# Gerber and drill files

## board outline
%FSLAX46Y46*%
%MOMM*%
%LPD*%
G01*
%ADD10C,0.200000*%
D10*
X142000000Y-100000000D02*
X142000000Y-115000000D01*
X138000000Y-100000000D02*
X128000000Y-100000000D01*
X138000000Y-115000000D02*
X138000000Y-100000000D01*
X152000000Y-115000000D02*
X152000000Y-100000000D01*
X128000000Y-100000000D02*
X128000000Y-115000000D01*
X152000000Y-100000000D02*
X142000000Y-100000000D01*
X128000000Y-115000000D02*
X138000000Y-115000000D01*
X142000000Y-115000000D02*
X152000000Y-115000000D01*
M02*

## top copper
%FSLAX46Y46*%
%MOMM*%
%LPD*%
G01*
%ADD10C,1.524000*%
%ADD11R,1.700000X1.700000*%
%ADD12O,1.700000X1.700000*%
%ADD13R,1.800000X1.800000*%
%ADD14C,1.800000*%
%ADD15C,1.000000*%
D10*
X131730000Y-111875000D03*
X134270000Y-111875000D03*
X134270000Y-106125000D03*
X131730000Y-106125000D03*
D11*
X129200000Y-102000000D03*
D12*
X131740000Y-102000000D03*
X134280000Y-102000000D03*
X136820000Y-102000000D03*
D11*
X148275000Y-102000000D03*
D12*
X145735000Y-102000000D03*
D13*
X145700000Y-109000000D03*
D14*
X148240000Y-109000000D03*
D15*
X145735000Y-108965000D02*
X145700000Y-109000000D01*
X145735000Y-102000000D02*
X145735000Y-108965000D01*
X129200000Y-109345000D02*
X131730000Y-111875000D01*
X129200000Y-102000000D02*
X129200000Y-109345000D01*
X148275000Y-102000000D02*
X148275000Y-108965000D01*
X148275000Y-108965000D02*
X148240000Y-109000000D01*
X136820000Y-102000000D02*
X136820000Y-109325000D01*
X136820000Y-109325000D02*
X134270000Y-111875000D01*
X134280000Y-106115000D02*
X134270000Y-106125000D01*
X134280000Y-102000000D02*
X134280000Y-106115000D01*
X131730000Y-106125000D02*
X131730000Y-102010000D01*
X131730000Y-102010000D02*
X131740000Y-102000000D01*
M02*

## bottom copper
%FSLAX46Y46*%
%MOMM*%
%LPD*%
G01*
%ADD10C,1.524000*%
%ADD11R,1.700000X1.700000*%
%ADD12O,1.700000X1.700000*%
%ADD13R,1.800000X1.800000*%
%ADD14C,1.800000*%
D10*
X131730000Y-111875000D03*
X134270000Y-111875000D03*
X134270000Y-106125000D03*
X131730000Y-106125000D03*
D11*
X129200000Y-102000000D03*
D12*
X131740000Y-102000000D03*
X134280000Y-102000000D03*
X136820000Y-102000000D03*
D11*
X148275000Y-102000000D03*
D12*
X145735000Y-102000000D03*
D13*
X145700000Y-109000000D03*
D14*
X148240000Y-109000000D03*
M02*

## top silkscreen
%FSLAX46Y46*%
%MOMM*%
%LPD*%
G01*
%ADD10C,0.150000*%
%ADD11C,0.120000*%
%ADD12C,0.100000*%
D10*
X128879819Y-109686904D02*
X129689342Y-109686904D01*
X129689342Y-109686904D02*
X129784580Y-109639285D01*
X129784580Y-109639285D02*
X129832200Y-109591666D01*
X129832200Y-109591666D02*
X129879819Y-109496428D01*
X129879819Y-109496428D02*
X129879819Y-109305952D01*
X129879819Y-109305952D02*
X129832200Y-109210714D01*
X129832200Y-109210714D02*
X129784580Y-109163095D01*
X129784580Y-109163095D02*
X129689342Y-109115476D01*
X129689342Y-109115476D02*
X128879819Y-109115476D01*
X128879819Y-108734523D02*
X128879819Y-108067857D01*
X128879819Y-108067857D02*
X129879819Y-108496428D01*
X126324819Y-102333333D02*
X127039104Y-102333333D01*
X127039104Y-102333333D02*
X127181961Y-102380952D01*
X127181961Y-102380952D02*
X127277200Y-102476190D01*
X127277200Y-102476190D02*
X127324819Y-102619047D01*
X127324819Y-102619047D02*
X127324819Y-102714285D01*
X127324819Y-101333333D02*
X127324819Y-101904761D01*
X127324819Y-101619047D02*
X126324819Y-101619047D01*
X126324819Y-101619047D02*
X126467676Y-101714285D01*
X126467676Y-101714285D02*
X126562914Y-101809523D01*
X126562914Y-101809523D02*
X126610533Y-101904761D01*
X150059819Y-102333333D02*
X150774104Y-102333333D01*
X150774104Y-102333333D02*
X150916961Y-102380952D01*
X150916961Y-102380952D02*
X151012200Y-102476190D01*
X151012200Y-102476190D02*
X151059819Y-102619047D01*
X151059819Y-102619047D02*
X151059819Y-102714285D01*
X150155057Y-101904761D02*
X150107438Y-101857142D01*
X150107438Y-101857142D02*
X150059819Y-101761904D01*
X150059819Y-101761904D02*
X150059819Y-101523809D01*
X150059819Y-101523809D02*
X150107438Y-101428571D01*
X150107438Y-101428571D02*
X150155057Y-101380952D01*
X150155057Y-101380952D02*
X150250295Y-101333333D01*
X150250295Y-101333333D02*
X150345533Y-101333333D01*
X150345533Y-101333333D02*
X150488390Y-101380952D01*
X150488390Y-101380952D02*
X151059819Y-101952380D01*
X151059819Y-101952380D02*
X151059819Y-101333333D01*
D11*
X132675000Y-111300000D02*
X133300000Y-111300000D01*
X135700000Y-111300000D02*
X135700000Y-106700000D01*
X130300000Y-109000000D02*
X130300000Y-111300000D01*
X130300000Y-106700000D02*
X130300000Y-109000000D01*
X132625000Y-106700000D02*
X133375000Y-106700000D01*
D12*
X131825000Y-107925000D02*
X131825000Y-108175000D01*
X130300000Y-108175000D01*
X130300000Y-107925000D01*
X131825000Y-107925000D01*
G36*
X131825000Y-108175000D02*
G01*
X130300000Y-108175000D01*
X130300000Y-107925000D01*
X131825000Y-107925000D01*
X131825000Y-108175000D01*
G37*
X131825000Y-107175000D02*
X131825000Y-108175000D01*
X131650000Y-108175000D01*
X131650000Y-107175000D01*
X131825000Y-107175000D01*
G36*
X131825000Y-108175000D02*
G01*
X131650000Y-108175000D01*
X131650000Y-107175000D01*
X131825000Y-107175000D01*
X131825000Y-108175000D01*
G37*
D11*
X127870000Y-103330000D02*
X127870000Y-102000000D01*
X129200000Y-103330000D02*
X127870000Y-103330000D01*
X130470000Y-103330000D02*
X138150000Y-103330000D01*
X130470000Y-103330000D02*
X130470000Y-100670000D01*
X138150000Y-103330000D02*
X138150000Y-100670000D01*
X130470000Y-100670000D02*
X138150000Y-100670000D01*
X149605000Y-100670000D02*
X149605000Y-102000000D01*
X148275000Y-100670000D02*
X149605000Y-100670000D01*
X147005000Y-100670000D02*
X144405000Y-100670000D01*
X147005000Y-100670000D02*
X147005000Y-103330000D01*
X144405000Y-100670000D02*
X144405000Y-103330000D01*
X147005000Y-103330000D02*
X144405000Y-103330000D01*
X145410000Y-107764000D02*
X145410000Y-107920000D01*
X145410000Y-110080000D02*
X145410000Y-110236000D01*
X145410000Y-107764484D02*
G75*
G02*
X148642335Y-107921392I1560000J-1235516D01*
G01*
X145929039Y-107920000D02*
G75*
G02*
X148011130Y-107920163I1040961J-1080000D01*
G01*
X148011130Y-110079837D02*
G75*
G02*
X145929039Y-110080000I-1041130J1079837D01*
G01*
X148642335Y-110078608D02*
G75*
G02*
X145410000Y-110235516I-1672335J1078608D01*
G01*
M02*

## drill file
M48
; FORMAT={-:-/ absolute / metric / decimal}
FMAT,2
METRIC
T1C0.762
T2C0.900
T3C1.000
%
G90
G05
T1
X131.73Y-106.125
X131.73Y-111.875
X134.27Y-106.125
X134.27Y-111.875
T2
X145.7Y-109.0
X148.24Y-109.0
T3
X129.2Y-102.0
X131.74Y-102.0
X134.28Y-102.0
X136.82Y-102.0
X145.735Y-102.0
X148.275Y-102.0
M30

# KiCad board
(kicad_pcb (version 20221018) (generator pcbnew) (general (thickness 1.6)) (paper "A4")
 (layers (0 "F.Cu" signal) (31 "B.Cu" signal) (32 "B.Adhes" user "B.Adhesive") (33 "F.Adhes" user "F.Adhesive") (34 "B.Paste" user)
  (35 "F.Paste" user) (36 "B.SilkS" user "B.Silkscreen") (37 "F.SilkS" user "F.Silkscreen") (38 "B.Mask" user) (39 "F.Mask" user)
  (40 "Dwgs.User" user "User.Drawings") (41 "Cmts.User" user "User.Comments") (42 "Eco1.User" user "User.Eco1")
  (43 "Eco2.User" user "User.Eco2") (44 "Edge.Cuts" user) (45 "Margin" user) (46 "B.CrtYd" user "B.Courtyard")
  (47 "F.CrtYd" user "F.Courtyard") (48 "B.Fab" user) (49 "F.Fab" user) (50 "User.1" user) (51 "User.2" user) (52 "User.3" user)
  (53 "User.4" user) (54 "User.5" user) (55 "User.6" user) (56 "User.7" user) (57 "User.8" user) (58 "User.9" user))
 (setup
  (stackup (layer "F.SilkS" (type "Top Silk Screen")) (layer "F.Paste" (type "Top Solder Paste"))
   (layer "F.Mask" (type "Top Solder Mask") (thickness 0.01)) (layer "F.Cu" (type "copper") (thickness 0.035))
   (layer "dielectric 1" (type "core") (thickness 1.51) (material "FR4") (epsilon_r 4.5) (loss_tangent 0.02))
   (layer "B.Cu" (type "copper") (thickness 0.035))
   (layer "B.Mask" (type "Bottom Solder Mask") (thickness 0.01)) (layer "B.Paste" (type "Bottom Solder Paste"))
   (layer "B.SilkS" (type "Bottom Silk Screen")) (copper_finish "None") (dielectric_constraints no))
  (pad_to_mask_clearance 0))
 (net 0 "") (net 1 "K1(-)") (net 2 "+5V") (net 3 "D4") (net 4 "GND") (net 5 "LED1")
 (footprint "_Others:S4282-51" (layer "F.Cu") (at 133 109 90)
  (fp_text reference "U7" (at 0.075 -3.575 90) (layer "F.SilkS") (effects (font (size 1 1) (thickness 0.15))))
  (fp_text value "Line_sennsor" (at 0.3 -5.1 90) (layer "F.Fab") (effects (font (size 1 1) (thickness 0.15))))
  (fp_line (start -2.3 -0.325) (end -2.3 0.3) (stroke (width 0.12) (type solid)) (layer "F.SilkS"))
  (fp_line (start -2.3 2.7) (end 2.3 2.7) (stroke (width 0.12) (type solid)) (layer "F.SilkS"))
  (fp_line (start 0 -2.7) (end -2.3 -2.7) (stroke (width 0.12) (type solid)) (layer "F.SilkS"))
  (fp_line (start 2.3 -2.7) (end 0 -2.7) (stroke (width 0.12) (type solid)) (layer "F.SilkS"))
  (fp_line (start 2.3 -0.375) (end 2.3 0.375) (stroke (width 0.12) (type solid)) (layer "F.SilkS"))
  (fp_poly
   (pts (xy 1.075 -1.175) (xy 0.825 -1.175) (xy 0.825 -2.7) (xy 1.075 -2.7)) (stroke (width 0.1) (type solid)) (fill solid)
   (layer "F.SilkS"))
  (fp_poly
   (pts (xy 1.825 -1.175) (xy 0.825 -1.175) (xy 0.825 -1.35) (xy 1.825 -1.35)) (stroke (width 0.1) (type solid)) (fill solid)
   (layer "F.SilkS"))
  (pad "1" thru_hole circle (at -2.875 -1.27 90) (size 1.524 1.524) (drill 0.762) (layers "*.Cu" "*.Mask") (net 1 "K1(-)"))
  (pad "2" thru_hole circle (at -2.875 1.27 90) (size 1.524 1.524) (drill 0.762) (layers "*.Cu" "*.Mask") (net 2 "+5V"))
  (pad "3" thru_hole circle (at 2.875 1.27 90) (size 1.524 1.524) (drill 0.762) (layers "*.Cu" "*.Mask") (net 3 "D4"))
  (pad "4" thru_hole circle (at 2.875 -1.27 90) (size 1.524 1.524) (drill 0.762) (layers "*.Cu" "*.Mask") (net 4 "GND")))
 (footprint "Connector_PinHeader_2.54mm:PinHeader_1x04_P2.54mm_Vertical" (layer "F.Cu") (at 129.2 102 90)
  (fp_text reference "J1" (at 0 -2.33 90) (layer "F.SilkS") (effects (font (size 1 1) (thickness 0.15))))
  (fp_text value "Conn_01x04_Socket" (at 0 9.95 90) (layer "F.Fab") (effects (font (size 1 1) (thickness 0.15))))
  (fp_line (start -1.33 -1.33) (end 0 -1.33) (stroke (width 0.12) (type solid)) (layer "F.SilkS"))
  (fp_line (start -1.33 0) (end -1.33 -1.33) (stroke (width 0.12) (type solid)) (layer "F.SilkS"))
  (fp_line (start -1.33 1.27) (end -1.33 8.95) (stroke (width 0.12) (type solid)) (layer "F.SilkS"))
  (fp_line (start -1.33 1.27) (end 1.33 1.27) (stroke (width 0.12) (type solid)) (layer "F.SilkS"))
  (fp_line (start -1.33 8.95) (end 1.33 8.95) (stroke (width 0.12) (type solid)) (layer "F.SilkS"))
  (fp_line (start 1.33 1.27) (end 1.33 8.95) (stroke (width 0.12) (type solid)) (layer "F.SilkS"))
  (pad "1" thru_hole rect (at 0 0 90) (size 1.7 1.7) (drill 1) (layers "*.Cu" "*.Mask") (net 1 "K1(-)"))
  (pad "2" thru_hole oval (at 0 2.54 90) (size 1.7 1.7) (drill 1) (layers "*.Cu" "*.Mask") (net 4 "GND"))
  (pad "3" thru_hole oval (at 0 5.08 90) (size 1.7 1.7) (drill 1) (layers "*.Cu" "*.Mask") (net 3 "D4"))
  (pad "4" thru_hole oval (at 0 7.62 90) (size 1.7 1.7) (drill 1) (layers "*.Cu" "*.Mask") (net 2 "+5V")))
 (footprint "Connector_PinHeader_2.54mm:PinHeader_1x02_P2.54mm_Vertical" (layer "F.Cu") (at 148.275 102 -90)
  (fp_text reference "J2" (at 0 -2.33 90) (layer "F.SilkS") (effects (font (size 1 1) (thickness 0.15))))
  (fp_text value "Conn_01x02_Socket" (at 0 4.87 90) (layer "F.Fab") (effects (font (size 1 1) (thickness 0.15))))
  (fp_line (start -1.33 -1.33) (end 0 -1.33) (stroke (width 0.12) (type solid)) (layer "F.SilkS"))
  (fp_line (start -1.33 0) (end -1.33 -1.33) (stroke (width 0.12) (type solid)) (layer "F.SilkS"))
  (fp_line (start -1.33 1.27) (end -1.33 3.87) (stroke (width 0.12) (type solid)) (layer "F.SilkS"))
  (fp_line (start -1.33 1.27) (end 1.33 1.27) (stroke (width 0.12) (type solid)) (layer "F.SilkS"))
  (fp_line (start -1.33 3.87) (end 1.33 3.87) (stroke (width 0.12) (type solid)) (layer "F.SilkS"))
  (fp_line (start 1.33 1.27) (end 1.33 3.87) (stroke (width 0.12) (type solid)) (layer "F.SilkS"))
  (pad "1" thru_hole rect (at 0 0 270) (size 1.7 1.7) (drill 1) (layers "*.Cu" "*.Mask") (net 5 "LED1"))
  (pad "2" thru_hole oval (at 0 2.54 270) (size 1.7 1.7) (drill 1) (layers "*.Cu" "*.Mask") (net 1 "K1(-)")))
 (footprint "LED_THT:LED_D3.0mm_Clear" (layer "F.Cu") (at 145.7 109)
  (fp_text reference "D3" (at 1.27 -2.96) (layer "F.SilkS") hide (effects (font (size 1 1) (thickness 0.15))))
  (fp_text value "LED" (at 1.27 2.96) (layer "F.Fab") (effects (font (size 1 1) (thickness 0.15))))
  (fp_line (start -0.29 -1.236) (end -0.29 -1.08) (stroke (width 0.12) (type solid)) (layer "F.SilkS"))
  (fp_line (start -0.29 1.08) (end -0.29 1.236) (stroke (width 0.12) (type solid)) (layer "F.SilkS"))
  (fp_arc (start -0.29 -1.235516) (mid 1.366487 -1.987659) (end 2.942335 -1.078608) (stroke (width 0.12) (type solid)) (layer "F.SilkS"))
  (fp_arc (start 0.229039 -1.08) (mid 1.270117 -1.5) (end 2.31113 -1.079837) (stroke (width 0.12) (type solid)) (layer "F.SilkS"))
  (fp_arc (start 2.31113 1.079837) (mid 1.270117 1.5) (end 0.229039 1.08) (stroke (width 0.12) (type solid)) (layer "F.SilkS"))
  (fp_arc (start 2.942335 1.078608) (mid 1.366487 1.987659) (end -0.29 1.235516) (stroke (width 0.12) (type solid)) (layer "F.SilkS"))
  (pad "1" thru_hole rect (at 0 0) (size 1.8 1.8) (drill 0.9) (layers "*.Cu" "*.Mask") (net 1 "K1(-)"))
  (pad "2" thru_hole circle (at 2.54 0) (size 1.8 1.8) (drill 0.9) (layers "*.Cu" "*.Mask") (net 5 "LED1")))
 (gr_line (start 142 100) (end 142 115) (stroke (width 0.2) (type solid)) (layer "Edge.Cuts"))
 (gr_line (start 138 100) (end 128 100) (stroke (width 0.2) (type solid)) (layer "Edge.Cuts"))
 (gr_line (start 138 115) (end 138 100) (stroke (width 0.2) (type solid)) (layer "Edge.Cuts"))
 (gr_line (start 152 115) (end 152 100) (stroke (width 0.2) (type solid)) (layer "Edge.Cuts"))
 (gr_line (start 128 100) (end 128 115) (stroke (width 0.2) (type solid)) (layer "Edge.Cuts"))
 (gr_line (start 152 100) (end 142 100) (stroke (width 0.2) (type solid)) (layer "Edge.Cuts"))
 (gr_line (start 128 115) (end 138 115) (stroke (width 0.2) (type solid)) (layer "Edge.Cuts"))
 (gr_line (start 142 115) (end 152 115) (stroke (width 0.2) (type solid)) (layer "Edge.Cuts"))
 (segment (start 145.735 108.965) (end 145.7 109) (width 1) (layer "F.Cu") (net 1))
 (segment (start 145.735 102) (end 145.735 108.965) (width 1) (layer "F.Cu") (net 1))
 (segment (start 129.2 109.345) (end 131.73 111.875) (width 1) (layer "F.Cu") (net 1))
 (segment (start 129.2 102) (end 129.2 109.345) (width 1) (layer "F.Cu") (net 1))
 (segment (start 148.275 102) (end 148.275 108.965) (width 1) (layer "F.Cu") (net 5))
 (segment (start 148.275 108.965) (end 148.24 109) (width 1) (layer "F.Cu") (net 5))
 (segment (start 136.82 102) (end 136.82 109.325) (width 1) (layer "F.Cu") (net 2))
 (segment (start 136.82 109.325) (end 134.27 111.875) (width 1) (layer "F.Cu") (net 2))
 (segment (start 134.28 106.115) (end 134.27 106.125) (width 1) (layer "F.Cu") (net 3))
 (segment (start 134.28 102) (end 134.28 106.115) (width 1) (layer "F.Cu") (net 3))
 (segment (start 131.73 106.125) (end 131.73 102.01) (width 1) (layer "F.Cu") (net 4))
 (segment (start 131.73 102.01) (end 131.74 102) (width 1) (layer "F.Cu") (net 4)))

